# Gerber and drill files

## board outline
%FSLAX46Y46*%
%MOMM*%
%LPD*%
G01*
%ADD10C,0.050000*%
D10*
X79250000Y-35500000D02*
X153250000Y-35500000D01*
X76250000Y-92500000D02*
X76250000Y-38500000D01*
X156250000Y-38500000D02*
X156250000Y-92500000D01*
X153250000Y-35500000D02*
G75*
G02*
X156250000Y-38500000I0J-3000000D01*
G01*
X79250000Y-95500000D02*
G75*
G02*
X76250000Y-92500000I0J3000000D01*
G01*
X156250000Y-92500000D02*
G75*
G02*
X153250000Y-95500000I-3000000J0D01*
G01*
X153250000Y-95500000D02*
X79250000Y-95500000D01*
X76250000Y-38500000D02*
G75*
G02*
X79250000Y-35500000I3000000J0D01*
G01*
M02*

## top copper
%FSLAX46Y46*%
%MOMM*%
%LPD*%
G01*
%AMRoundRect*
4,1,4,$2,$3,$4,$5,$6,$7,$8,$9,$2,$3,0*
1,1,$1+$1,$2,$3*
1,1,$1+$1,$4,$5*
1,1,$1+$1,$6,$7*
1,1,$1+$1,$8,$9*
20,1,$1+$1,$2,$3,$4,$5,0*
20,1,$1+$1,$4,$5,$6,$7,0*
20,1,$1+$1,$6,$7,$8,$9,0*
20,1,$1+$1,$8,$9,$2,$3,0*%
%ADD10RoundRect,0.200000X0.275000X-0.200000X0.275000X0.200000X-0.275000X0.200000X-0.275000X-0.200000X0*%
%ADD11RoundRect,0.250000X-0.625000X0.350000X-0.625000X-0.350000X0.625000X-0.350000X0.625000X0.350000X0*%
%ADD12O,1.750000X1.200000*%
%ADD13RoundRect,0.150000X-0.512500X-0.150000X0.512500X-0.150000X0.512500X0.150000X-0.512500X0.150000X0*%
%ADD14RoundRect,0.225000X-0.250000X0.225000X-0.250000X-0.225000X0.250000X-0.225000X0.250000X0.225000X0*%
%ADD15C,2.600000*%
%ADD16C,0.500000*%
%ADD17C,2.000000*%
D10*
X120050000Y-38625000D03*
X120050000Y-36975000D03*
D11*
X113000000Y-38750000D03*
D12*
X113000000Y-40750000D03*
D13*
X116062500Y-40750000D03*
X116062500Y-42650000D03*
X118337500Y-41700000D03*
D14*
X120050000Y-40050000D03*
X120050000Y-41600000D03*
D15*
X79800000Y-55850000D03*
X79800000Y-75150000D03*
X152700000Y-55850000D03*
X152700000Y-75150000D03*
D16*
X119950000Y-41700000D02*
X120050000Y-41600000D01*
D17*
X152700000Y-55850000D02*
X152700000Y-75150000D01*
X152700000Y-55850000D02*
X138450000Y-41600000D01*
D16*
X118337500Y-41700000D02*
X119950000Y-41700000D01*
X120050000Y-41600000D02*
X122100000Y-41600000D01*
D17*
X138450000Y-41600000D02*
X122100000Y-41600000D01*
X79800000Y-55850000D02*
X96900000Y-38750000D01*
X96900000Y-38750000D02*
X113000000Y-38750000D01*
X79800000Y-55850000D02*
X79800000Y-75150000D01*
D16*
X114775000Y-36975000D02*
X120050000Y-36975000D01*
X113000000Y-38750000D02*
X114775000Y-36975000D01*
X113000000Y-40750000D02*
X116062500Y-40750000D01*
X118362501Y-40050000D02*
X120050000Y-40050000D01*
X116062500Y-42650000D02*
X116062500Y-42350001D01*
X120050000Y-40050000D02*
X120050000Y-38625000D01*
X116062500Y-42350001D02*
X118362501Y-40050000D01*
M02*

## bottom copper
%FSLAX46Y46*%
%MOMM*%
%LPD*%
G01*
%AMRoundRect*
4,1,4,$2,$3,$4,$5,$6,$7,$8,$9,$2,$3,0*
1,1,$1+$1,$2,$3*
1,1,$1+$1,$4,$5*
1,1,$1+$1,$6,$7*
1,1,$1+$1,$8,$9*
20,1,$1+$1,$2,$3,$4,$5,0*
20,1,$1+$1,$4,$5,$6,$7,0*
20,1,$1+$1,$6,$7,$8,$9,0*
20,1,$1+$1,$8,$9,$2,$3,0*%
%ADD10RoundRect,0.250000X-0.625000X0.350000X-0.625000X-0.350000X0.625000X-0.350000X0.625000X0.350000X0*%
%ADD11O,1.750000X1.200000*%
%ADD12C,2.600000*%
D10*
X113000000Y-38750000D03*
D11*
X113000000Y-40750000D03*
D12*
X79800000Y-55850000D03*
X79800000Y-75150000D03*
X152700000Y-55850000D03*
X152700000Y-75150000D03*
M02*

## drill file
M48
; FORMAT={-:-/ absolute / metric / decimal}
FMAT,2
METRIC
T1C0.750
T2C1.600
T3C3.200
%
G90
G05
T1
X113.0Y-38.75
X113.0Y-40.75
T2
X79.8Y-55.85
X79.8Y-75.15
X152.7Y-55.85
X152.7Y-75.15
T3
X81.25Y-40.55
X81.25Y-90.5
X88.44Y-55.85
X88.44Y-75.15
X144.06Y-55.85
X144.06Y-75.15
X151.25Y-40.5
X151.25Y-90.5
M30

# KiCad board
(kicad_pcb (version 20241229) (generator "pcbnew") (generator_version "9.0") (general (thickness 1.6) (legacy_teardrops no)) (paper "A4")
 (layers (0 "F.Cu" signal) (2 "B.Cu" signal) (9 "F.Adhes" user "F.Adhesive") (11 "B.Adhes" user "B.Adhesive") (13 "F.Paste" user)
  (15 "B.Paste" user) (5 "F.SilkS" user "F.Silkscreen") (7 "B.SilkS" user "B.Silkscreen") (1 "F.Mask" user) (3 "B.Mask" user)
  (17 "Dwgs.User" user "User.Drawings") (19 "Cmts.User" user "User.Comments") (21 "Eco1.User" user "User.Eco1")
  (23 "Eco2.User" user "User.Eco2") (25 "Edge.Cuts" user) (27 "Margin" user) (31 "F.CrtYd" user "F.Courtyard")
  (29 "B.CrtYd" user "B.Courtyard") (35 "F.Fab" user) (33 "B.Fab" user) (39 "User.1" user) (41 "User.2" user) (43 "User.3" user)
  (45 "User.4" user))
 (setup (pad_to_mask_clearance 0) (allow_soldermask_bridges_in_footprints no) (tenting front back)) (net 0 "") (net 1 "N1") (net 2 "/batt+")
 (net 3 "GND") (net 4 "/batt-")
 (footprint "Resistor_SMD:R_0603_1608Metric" (layer "F.Cu") (at 120.05 37.8 90)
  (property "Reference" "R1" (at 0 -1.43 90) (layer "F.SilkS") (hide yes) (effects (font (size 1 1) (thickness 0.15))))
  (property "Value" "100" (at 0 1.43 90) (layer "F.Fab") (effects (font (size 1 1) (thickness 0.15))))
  (pad "1" smd roundrect (at -0.825 0 90) (size 0.8 0.95) (layers "F.Cu" "F.Mask" "F.Paste") (roundrect_rratio 0.25) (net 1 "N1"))
  (pad "2" smd roundrect (at 0.825 0 90) (size 0.8 0.95) (layers "F.Cu" "F.Mask" "F.Paste") (roundrect_rratio 0.25) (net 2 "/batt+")))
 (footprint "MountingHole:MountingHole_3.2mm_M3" (layer "F.Cu") (at 151.25 40.5)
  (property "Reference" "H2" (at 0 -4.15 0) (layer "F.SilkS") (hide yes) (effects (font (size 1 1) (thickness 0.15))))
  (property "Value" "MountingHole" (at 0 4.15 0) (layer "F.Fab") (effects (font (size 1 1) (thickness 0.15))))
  (pad "" np_thru_hole circle (at 0 0) (size 3.2 3.2) (drill 3.2) (layers "*.Cu" "*.Mask")))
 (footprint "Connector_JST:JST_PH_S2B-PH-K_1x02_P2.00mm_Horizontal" (layer "F.Cu") (at 113 38.75 -90)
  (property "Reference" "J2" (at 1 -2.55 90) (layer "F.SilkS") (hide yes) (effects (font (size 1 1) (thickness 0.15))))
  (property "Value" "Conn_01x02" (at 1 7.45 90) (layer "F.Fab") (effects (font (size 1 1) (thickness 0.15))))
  (pad "1" thru_hole roundrect (at 0 0 270) (size 1.2 1.75) (drill 0.75) (layers "*.Cu" "*.Mask") (remove_unused_layers no)
   (roundrect_rratio 0.208333) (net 2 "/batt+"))
  (pad "2" thru_hole oval (at 2 0 270) (size 1.2 1.75) (drill 0.75) (layers "*.Cu" "*.Mask") (remove_unused_layers no) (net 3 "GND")))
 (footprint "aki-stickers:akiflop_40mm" (layer "F.Cu") (at 114.45 63.9)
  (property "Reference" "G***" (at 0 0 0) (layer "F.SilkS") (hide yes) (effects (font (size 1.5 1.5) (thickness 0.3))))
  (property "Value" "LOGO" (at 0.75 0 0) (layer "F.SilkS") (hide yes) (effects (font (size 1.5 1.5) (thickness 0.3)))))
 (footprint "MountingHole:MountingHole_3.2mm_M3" (layer "F.Cu") (at 81.25 40.55)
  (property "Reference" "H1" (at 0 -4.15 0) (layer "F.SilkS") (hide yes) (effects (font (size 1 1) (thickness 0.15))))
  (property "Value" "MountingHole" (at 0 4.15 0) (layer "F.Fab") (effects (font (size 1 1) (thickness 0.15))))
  (pad "" np_thru_hole circle (at 0 0) (size 3.2 3.2) (drill 3.2) (layers "*.Cu" "*.Mask")))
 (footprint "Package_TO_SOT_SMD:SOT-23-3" (layer "F.Cu") (at 117.2 41.7)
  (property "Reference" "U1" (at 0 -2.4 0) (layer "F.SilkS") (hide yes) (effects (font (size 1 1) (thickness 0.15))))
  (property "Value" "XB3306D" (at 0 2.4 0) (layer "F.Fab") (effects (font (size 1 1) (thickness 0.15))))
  (pad "1" smd roundrect (at -1.1375 -0.95) (size 1.325 0.6) (layers "F.Cu" "F.Mask" "F.Paste") (roundrect_rratio 0.25) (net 3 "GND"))
  (pad "2" smd roundrect (at -1.1375 0.95) (size 1.325 0.6) (layers "F.Cu" "F.Mask" "F.Paste") (roundrect_rratio 0.25) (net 1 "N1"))
  (pad "3" smd roundrect (at 1.1375 0) (size 1.325 0.6) (layers "F.Cu" "F.Mask" "F.Paste") (roundrect_rratio 0.25) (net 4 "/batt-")))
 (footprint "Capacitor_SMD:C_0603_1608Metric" (layer "F.Cu") (at 120.05 40.825 -90)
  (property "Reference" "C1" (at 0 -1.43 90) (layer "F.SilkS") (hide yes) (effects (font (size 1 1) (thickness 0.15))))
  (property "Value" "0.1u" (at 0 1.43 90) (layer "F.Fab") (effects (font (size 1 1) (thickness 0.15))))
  (pad "1" smd roundrect (at -0.775 0 270) (size 0.9 0.95) (layers "F.Cu" "F.Mask" "F.Paste") (roundrect_rratio 0.25) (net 1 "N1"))
  (pad "2" smd roundrect (at 0.775 0 270) (size 0.9 0.95) (layers "F.Cu" "F.Mask" "F.Paste") (roundrect_rratio 0.25) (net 4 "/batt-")))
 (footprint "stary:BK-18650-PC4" (layer "F.Cu") (at 116.25 65.5)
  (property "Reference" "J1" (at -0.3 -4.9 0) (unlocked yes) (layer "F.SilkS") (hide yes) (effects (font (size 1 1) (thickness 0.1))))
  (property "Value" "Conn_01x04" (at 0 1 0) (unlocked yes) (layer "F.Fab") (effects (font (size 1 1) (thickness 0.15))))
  (pad "" np_thru_hole circle (at -27.81 -9.65) (size 3.2 3.2) (drill 3.2) (layers "*.Cu" "*.Mask"))
  (pad "" np_thru_hole circle (at -27.81 9.65) (size 3.2 3.2) (drill 3.2) (layers "*.Cu" "*.Mask"))
  (pad "" np_thru_hole circle (at 27.81 -9.65) (size 3.2 3.2) (drill 3.2) (layers "*.Cu" "*.Mask"))
  (pad "" np_thru_hole circle (at 27.81 9.65) (size 3.2 3.2) (drill 3.2) (layers "*.Cu" "*.Mask"))
  (pad "1" thru_hole circle (at -36.45 -9.65) (size 2.6 2.6) (drill 1.6) (layers "*.Cu" "*.Mask") (remove_unused_layers no) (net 2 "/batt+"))
  (pad "2" thru_hole circle (at -36.45 9.65) (size 2.6 2.6) (drill 1.6) (layers "*.Cu" "*.Mask") (remove_unused_layers no) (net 2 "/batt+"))
  (pad "3" thru_hole circle (at 36.45 -9.65) (size 2.6 2.6) (drill 1.6) (layers "*.Cu" "*.Mask") (remove_unused_layers no) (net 4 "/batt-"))
  (pad "4" thru_hole circle (at 36.45 9.65) (size 2.6 2.6) (drill 1.6) (layers "*.Cu" "*.Mask") (remove_unused_layers no) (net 4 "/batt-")))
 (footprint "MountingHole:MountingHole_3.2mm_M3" (layer "F.Cu") (at 151.25 90.5)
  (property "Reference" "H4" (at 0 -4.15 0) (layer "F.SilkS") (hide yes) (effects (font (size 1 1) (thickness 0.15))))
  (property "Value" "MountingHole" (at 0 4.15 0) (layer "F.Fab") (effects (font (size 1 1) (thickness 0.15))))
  (pad "" np_thru_hole circle (at 0 0) (size 3.2 3.2) (drill 3.2) (layers "*.Cu" "*.Mask")))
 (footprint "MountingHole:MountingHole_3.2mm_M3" (layer "F.Cu") (at 81.25 90.5)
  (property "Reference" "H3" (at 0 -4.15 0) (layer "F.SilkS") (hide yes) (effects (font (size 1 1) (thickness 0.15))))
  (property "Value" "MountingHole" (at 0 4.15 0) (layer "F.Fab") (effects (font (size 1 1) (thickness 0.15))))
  (pad "" np_thru_hole circle (at 0 0) (size 3.2 3.2) (drill 3.2) (layers "*.Cu" "*.Mask")))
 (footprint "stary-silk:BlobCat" (layer "B.Cu") (at 116.262871 65.590097 180)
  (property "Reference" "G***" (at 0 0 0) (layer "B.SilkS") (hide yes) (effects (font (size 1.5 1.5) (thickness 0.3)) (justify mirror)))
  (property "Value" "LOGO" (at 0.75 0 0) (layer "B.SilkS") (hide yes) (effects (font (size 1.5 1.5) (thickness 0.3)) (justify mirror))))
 (gr_line (start 79.25 35.5) (end 153.25 35.5) (stroke (width 0.05) (type default)) (layer "Edge.Cuts"))
 (gr_line (start 76.25 92.5) (end 76.25 38.5) (stroke (width 0.05) (type default)) (layer "Edge.Cuts"))
 (gr_line (start 156.25 38.5) (end 156.25 92.5) (stroke (width 0.05) (type default)) (layer "Edge.Cuts"))
 (gr_arc (start 153.25 35.5) (mid 155.37132 36.37868) (end 156.25 38.5) (stroke (width 0.05) (type default)) (layer "Edge.Cuts"))
 (gr_arc (start 79.25 95.5) (mid 77.12868 94.62132) (end 76.25 92.5) (stroke (width 0.05) (type default)) (layer "Edge.Cuts"))
 (gr_arc (start 156.25 92.5) (mid 155.37132 94.62132) (end 153.25 95.5) (stroke (width 0.05) (type default)) (layer "Edge.Cuts"))
 (gr_line (start 153.25 95.5) (end 79.25 95.5) (stroke (width 0.05) (type default)) (layer "Edge.Cuts"))
 (gr_arc (start 76.25 38.5) (mid 77.12868 36.37868) (end 79.25 35.5) (stroke (width 0.05) (type default)) (layer "Edge.Cuts"))
 (segment (start 119.95 41.7) (end 120.05 41.6) (width 0.5) (layer "F.Cu") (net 4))
 (segment (start 152.7 55.85) (end 152.7 75.15) (width 2) (layer "F.Cu") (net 4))
 (segment (start 152.7 55.85) (end 138.45 41.6) (width 2) (layer "F.Cu") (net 4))
 (segment (start 118.3375 41.7) (end 119.95 41.7) (width 0.5) (layer "F.Cu") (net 4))
 (segment (start 120.05 41.6) (end 122.1 41.6) (width 0.5) (layer "F.Cu") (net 4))
 (segment (start 138.45 41.6) (end 122.1 41.6) (width 2) (layer "F.Cu") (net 4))
 (segment (start 79.8 55.85) (end 96.9 38.75) (width 2) (layer "F.Cu") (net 2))
 (segment (start 96.9 38.75) (end 113 38.75) (width 2) (layer "F.Cu") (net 2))
 (segment (start 79.8 55.85) (end 79.8 75.15) (width 2) (layer "F.Cu") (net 2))
 (segment (start 114.775 36.975) (end 120.05 36.975) (width 0.5) (layer "F.Cu") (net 2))
 (segment (start 113 38.75) (end 114.775 36.975) (width 0.5) (layer "F.Cu") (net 2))
 (segment (start 113 40.75) (end 116.0625 40.75) (width 0.5) (layer "F.Cu") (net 3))
 (segment (start 118.362501 40.05) (end 120.05 40.05) (width 0.5) (layer "F.Cu") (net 1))
 (segment (start 116.0625 42.65) (end 116.0625 42.350001) (width 0.5) (layer "F.Cu") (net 1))
 (segment (start 120.05 40.05) (end 120.05 38.625) (width 0.5) (layer "F.Cu") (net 1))
 (segment (start 116.0625 42.350001) (end 118.362501 40.05) (width 0.5) (layer "F.Cu") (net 1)))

